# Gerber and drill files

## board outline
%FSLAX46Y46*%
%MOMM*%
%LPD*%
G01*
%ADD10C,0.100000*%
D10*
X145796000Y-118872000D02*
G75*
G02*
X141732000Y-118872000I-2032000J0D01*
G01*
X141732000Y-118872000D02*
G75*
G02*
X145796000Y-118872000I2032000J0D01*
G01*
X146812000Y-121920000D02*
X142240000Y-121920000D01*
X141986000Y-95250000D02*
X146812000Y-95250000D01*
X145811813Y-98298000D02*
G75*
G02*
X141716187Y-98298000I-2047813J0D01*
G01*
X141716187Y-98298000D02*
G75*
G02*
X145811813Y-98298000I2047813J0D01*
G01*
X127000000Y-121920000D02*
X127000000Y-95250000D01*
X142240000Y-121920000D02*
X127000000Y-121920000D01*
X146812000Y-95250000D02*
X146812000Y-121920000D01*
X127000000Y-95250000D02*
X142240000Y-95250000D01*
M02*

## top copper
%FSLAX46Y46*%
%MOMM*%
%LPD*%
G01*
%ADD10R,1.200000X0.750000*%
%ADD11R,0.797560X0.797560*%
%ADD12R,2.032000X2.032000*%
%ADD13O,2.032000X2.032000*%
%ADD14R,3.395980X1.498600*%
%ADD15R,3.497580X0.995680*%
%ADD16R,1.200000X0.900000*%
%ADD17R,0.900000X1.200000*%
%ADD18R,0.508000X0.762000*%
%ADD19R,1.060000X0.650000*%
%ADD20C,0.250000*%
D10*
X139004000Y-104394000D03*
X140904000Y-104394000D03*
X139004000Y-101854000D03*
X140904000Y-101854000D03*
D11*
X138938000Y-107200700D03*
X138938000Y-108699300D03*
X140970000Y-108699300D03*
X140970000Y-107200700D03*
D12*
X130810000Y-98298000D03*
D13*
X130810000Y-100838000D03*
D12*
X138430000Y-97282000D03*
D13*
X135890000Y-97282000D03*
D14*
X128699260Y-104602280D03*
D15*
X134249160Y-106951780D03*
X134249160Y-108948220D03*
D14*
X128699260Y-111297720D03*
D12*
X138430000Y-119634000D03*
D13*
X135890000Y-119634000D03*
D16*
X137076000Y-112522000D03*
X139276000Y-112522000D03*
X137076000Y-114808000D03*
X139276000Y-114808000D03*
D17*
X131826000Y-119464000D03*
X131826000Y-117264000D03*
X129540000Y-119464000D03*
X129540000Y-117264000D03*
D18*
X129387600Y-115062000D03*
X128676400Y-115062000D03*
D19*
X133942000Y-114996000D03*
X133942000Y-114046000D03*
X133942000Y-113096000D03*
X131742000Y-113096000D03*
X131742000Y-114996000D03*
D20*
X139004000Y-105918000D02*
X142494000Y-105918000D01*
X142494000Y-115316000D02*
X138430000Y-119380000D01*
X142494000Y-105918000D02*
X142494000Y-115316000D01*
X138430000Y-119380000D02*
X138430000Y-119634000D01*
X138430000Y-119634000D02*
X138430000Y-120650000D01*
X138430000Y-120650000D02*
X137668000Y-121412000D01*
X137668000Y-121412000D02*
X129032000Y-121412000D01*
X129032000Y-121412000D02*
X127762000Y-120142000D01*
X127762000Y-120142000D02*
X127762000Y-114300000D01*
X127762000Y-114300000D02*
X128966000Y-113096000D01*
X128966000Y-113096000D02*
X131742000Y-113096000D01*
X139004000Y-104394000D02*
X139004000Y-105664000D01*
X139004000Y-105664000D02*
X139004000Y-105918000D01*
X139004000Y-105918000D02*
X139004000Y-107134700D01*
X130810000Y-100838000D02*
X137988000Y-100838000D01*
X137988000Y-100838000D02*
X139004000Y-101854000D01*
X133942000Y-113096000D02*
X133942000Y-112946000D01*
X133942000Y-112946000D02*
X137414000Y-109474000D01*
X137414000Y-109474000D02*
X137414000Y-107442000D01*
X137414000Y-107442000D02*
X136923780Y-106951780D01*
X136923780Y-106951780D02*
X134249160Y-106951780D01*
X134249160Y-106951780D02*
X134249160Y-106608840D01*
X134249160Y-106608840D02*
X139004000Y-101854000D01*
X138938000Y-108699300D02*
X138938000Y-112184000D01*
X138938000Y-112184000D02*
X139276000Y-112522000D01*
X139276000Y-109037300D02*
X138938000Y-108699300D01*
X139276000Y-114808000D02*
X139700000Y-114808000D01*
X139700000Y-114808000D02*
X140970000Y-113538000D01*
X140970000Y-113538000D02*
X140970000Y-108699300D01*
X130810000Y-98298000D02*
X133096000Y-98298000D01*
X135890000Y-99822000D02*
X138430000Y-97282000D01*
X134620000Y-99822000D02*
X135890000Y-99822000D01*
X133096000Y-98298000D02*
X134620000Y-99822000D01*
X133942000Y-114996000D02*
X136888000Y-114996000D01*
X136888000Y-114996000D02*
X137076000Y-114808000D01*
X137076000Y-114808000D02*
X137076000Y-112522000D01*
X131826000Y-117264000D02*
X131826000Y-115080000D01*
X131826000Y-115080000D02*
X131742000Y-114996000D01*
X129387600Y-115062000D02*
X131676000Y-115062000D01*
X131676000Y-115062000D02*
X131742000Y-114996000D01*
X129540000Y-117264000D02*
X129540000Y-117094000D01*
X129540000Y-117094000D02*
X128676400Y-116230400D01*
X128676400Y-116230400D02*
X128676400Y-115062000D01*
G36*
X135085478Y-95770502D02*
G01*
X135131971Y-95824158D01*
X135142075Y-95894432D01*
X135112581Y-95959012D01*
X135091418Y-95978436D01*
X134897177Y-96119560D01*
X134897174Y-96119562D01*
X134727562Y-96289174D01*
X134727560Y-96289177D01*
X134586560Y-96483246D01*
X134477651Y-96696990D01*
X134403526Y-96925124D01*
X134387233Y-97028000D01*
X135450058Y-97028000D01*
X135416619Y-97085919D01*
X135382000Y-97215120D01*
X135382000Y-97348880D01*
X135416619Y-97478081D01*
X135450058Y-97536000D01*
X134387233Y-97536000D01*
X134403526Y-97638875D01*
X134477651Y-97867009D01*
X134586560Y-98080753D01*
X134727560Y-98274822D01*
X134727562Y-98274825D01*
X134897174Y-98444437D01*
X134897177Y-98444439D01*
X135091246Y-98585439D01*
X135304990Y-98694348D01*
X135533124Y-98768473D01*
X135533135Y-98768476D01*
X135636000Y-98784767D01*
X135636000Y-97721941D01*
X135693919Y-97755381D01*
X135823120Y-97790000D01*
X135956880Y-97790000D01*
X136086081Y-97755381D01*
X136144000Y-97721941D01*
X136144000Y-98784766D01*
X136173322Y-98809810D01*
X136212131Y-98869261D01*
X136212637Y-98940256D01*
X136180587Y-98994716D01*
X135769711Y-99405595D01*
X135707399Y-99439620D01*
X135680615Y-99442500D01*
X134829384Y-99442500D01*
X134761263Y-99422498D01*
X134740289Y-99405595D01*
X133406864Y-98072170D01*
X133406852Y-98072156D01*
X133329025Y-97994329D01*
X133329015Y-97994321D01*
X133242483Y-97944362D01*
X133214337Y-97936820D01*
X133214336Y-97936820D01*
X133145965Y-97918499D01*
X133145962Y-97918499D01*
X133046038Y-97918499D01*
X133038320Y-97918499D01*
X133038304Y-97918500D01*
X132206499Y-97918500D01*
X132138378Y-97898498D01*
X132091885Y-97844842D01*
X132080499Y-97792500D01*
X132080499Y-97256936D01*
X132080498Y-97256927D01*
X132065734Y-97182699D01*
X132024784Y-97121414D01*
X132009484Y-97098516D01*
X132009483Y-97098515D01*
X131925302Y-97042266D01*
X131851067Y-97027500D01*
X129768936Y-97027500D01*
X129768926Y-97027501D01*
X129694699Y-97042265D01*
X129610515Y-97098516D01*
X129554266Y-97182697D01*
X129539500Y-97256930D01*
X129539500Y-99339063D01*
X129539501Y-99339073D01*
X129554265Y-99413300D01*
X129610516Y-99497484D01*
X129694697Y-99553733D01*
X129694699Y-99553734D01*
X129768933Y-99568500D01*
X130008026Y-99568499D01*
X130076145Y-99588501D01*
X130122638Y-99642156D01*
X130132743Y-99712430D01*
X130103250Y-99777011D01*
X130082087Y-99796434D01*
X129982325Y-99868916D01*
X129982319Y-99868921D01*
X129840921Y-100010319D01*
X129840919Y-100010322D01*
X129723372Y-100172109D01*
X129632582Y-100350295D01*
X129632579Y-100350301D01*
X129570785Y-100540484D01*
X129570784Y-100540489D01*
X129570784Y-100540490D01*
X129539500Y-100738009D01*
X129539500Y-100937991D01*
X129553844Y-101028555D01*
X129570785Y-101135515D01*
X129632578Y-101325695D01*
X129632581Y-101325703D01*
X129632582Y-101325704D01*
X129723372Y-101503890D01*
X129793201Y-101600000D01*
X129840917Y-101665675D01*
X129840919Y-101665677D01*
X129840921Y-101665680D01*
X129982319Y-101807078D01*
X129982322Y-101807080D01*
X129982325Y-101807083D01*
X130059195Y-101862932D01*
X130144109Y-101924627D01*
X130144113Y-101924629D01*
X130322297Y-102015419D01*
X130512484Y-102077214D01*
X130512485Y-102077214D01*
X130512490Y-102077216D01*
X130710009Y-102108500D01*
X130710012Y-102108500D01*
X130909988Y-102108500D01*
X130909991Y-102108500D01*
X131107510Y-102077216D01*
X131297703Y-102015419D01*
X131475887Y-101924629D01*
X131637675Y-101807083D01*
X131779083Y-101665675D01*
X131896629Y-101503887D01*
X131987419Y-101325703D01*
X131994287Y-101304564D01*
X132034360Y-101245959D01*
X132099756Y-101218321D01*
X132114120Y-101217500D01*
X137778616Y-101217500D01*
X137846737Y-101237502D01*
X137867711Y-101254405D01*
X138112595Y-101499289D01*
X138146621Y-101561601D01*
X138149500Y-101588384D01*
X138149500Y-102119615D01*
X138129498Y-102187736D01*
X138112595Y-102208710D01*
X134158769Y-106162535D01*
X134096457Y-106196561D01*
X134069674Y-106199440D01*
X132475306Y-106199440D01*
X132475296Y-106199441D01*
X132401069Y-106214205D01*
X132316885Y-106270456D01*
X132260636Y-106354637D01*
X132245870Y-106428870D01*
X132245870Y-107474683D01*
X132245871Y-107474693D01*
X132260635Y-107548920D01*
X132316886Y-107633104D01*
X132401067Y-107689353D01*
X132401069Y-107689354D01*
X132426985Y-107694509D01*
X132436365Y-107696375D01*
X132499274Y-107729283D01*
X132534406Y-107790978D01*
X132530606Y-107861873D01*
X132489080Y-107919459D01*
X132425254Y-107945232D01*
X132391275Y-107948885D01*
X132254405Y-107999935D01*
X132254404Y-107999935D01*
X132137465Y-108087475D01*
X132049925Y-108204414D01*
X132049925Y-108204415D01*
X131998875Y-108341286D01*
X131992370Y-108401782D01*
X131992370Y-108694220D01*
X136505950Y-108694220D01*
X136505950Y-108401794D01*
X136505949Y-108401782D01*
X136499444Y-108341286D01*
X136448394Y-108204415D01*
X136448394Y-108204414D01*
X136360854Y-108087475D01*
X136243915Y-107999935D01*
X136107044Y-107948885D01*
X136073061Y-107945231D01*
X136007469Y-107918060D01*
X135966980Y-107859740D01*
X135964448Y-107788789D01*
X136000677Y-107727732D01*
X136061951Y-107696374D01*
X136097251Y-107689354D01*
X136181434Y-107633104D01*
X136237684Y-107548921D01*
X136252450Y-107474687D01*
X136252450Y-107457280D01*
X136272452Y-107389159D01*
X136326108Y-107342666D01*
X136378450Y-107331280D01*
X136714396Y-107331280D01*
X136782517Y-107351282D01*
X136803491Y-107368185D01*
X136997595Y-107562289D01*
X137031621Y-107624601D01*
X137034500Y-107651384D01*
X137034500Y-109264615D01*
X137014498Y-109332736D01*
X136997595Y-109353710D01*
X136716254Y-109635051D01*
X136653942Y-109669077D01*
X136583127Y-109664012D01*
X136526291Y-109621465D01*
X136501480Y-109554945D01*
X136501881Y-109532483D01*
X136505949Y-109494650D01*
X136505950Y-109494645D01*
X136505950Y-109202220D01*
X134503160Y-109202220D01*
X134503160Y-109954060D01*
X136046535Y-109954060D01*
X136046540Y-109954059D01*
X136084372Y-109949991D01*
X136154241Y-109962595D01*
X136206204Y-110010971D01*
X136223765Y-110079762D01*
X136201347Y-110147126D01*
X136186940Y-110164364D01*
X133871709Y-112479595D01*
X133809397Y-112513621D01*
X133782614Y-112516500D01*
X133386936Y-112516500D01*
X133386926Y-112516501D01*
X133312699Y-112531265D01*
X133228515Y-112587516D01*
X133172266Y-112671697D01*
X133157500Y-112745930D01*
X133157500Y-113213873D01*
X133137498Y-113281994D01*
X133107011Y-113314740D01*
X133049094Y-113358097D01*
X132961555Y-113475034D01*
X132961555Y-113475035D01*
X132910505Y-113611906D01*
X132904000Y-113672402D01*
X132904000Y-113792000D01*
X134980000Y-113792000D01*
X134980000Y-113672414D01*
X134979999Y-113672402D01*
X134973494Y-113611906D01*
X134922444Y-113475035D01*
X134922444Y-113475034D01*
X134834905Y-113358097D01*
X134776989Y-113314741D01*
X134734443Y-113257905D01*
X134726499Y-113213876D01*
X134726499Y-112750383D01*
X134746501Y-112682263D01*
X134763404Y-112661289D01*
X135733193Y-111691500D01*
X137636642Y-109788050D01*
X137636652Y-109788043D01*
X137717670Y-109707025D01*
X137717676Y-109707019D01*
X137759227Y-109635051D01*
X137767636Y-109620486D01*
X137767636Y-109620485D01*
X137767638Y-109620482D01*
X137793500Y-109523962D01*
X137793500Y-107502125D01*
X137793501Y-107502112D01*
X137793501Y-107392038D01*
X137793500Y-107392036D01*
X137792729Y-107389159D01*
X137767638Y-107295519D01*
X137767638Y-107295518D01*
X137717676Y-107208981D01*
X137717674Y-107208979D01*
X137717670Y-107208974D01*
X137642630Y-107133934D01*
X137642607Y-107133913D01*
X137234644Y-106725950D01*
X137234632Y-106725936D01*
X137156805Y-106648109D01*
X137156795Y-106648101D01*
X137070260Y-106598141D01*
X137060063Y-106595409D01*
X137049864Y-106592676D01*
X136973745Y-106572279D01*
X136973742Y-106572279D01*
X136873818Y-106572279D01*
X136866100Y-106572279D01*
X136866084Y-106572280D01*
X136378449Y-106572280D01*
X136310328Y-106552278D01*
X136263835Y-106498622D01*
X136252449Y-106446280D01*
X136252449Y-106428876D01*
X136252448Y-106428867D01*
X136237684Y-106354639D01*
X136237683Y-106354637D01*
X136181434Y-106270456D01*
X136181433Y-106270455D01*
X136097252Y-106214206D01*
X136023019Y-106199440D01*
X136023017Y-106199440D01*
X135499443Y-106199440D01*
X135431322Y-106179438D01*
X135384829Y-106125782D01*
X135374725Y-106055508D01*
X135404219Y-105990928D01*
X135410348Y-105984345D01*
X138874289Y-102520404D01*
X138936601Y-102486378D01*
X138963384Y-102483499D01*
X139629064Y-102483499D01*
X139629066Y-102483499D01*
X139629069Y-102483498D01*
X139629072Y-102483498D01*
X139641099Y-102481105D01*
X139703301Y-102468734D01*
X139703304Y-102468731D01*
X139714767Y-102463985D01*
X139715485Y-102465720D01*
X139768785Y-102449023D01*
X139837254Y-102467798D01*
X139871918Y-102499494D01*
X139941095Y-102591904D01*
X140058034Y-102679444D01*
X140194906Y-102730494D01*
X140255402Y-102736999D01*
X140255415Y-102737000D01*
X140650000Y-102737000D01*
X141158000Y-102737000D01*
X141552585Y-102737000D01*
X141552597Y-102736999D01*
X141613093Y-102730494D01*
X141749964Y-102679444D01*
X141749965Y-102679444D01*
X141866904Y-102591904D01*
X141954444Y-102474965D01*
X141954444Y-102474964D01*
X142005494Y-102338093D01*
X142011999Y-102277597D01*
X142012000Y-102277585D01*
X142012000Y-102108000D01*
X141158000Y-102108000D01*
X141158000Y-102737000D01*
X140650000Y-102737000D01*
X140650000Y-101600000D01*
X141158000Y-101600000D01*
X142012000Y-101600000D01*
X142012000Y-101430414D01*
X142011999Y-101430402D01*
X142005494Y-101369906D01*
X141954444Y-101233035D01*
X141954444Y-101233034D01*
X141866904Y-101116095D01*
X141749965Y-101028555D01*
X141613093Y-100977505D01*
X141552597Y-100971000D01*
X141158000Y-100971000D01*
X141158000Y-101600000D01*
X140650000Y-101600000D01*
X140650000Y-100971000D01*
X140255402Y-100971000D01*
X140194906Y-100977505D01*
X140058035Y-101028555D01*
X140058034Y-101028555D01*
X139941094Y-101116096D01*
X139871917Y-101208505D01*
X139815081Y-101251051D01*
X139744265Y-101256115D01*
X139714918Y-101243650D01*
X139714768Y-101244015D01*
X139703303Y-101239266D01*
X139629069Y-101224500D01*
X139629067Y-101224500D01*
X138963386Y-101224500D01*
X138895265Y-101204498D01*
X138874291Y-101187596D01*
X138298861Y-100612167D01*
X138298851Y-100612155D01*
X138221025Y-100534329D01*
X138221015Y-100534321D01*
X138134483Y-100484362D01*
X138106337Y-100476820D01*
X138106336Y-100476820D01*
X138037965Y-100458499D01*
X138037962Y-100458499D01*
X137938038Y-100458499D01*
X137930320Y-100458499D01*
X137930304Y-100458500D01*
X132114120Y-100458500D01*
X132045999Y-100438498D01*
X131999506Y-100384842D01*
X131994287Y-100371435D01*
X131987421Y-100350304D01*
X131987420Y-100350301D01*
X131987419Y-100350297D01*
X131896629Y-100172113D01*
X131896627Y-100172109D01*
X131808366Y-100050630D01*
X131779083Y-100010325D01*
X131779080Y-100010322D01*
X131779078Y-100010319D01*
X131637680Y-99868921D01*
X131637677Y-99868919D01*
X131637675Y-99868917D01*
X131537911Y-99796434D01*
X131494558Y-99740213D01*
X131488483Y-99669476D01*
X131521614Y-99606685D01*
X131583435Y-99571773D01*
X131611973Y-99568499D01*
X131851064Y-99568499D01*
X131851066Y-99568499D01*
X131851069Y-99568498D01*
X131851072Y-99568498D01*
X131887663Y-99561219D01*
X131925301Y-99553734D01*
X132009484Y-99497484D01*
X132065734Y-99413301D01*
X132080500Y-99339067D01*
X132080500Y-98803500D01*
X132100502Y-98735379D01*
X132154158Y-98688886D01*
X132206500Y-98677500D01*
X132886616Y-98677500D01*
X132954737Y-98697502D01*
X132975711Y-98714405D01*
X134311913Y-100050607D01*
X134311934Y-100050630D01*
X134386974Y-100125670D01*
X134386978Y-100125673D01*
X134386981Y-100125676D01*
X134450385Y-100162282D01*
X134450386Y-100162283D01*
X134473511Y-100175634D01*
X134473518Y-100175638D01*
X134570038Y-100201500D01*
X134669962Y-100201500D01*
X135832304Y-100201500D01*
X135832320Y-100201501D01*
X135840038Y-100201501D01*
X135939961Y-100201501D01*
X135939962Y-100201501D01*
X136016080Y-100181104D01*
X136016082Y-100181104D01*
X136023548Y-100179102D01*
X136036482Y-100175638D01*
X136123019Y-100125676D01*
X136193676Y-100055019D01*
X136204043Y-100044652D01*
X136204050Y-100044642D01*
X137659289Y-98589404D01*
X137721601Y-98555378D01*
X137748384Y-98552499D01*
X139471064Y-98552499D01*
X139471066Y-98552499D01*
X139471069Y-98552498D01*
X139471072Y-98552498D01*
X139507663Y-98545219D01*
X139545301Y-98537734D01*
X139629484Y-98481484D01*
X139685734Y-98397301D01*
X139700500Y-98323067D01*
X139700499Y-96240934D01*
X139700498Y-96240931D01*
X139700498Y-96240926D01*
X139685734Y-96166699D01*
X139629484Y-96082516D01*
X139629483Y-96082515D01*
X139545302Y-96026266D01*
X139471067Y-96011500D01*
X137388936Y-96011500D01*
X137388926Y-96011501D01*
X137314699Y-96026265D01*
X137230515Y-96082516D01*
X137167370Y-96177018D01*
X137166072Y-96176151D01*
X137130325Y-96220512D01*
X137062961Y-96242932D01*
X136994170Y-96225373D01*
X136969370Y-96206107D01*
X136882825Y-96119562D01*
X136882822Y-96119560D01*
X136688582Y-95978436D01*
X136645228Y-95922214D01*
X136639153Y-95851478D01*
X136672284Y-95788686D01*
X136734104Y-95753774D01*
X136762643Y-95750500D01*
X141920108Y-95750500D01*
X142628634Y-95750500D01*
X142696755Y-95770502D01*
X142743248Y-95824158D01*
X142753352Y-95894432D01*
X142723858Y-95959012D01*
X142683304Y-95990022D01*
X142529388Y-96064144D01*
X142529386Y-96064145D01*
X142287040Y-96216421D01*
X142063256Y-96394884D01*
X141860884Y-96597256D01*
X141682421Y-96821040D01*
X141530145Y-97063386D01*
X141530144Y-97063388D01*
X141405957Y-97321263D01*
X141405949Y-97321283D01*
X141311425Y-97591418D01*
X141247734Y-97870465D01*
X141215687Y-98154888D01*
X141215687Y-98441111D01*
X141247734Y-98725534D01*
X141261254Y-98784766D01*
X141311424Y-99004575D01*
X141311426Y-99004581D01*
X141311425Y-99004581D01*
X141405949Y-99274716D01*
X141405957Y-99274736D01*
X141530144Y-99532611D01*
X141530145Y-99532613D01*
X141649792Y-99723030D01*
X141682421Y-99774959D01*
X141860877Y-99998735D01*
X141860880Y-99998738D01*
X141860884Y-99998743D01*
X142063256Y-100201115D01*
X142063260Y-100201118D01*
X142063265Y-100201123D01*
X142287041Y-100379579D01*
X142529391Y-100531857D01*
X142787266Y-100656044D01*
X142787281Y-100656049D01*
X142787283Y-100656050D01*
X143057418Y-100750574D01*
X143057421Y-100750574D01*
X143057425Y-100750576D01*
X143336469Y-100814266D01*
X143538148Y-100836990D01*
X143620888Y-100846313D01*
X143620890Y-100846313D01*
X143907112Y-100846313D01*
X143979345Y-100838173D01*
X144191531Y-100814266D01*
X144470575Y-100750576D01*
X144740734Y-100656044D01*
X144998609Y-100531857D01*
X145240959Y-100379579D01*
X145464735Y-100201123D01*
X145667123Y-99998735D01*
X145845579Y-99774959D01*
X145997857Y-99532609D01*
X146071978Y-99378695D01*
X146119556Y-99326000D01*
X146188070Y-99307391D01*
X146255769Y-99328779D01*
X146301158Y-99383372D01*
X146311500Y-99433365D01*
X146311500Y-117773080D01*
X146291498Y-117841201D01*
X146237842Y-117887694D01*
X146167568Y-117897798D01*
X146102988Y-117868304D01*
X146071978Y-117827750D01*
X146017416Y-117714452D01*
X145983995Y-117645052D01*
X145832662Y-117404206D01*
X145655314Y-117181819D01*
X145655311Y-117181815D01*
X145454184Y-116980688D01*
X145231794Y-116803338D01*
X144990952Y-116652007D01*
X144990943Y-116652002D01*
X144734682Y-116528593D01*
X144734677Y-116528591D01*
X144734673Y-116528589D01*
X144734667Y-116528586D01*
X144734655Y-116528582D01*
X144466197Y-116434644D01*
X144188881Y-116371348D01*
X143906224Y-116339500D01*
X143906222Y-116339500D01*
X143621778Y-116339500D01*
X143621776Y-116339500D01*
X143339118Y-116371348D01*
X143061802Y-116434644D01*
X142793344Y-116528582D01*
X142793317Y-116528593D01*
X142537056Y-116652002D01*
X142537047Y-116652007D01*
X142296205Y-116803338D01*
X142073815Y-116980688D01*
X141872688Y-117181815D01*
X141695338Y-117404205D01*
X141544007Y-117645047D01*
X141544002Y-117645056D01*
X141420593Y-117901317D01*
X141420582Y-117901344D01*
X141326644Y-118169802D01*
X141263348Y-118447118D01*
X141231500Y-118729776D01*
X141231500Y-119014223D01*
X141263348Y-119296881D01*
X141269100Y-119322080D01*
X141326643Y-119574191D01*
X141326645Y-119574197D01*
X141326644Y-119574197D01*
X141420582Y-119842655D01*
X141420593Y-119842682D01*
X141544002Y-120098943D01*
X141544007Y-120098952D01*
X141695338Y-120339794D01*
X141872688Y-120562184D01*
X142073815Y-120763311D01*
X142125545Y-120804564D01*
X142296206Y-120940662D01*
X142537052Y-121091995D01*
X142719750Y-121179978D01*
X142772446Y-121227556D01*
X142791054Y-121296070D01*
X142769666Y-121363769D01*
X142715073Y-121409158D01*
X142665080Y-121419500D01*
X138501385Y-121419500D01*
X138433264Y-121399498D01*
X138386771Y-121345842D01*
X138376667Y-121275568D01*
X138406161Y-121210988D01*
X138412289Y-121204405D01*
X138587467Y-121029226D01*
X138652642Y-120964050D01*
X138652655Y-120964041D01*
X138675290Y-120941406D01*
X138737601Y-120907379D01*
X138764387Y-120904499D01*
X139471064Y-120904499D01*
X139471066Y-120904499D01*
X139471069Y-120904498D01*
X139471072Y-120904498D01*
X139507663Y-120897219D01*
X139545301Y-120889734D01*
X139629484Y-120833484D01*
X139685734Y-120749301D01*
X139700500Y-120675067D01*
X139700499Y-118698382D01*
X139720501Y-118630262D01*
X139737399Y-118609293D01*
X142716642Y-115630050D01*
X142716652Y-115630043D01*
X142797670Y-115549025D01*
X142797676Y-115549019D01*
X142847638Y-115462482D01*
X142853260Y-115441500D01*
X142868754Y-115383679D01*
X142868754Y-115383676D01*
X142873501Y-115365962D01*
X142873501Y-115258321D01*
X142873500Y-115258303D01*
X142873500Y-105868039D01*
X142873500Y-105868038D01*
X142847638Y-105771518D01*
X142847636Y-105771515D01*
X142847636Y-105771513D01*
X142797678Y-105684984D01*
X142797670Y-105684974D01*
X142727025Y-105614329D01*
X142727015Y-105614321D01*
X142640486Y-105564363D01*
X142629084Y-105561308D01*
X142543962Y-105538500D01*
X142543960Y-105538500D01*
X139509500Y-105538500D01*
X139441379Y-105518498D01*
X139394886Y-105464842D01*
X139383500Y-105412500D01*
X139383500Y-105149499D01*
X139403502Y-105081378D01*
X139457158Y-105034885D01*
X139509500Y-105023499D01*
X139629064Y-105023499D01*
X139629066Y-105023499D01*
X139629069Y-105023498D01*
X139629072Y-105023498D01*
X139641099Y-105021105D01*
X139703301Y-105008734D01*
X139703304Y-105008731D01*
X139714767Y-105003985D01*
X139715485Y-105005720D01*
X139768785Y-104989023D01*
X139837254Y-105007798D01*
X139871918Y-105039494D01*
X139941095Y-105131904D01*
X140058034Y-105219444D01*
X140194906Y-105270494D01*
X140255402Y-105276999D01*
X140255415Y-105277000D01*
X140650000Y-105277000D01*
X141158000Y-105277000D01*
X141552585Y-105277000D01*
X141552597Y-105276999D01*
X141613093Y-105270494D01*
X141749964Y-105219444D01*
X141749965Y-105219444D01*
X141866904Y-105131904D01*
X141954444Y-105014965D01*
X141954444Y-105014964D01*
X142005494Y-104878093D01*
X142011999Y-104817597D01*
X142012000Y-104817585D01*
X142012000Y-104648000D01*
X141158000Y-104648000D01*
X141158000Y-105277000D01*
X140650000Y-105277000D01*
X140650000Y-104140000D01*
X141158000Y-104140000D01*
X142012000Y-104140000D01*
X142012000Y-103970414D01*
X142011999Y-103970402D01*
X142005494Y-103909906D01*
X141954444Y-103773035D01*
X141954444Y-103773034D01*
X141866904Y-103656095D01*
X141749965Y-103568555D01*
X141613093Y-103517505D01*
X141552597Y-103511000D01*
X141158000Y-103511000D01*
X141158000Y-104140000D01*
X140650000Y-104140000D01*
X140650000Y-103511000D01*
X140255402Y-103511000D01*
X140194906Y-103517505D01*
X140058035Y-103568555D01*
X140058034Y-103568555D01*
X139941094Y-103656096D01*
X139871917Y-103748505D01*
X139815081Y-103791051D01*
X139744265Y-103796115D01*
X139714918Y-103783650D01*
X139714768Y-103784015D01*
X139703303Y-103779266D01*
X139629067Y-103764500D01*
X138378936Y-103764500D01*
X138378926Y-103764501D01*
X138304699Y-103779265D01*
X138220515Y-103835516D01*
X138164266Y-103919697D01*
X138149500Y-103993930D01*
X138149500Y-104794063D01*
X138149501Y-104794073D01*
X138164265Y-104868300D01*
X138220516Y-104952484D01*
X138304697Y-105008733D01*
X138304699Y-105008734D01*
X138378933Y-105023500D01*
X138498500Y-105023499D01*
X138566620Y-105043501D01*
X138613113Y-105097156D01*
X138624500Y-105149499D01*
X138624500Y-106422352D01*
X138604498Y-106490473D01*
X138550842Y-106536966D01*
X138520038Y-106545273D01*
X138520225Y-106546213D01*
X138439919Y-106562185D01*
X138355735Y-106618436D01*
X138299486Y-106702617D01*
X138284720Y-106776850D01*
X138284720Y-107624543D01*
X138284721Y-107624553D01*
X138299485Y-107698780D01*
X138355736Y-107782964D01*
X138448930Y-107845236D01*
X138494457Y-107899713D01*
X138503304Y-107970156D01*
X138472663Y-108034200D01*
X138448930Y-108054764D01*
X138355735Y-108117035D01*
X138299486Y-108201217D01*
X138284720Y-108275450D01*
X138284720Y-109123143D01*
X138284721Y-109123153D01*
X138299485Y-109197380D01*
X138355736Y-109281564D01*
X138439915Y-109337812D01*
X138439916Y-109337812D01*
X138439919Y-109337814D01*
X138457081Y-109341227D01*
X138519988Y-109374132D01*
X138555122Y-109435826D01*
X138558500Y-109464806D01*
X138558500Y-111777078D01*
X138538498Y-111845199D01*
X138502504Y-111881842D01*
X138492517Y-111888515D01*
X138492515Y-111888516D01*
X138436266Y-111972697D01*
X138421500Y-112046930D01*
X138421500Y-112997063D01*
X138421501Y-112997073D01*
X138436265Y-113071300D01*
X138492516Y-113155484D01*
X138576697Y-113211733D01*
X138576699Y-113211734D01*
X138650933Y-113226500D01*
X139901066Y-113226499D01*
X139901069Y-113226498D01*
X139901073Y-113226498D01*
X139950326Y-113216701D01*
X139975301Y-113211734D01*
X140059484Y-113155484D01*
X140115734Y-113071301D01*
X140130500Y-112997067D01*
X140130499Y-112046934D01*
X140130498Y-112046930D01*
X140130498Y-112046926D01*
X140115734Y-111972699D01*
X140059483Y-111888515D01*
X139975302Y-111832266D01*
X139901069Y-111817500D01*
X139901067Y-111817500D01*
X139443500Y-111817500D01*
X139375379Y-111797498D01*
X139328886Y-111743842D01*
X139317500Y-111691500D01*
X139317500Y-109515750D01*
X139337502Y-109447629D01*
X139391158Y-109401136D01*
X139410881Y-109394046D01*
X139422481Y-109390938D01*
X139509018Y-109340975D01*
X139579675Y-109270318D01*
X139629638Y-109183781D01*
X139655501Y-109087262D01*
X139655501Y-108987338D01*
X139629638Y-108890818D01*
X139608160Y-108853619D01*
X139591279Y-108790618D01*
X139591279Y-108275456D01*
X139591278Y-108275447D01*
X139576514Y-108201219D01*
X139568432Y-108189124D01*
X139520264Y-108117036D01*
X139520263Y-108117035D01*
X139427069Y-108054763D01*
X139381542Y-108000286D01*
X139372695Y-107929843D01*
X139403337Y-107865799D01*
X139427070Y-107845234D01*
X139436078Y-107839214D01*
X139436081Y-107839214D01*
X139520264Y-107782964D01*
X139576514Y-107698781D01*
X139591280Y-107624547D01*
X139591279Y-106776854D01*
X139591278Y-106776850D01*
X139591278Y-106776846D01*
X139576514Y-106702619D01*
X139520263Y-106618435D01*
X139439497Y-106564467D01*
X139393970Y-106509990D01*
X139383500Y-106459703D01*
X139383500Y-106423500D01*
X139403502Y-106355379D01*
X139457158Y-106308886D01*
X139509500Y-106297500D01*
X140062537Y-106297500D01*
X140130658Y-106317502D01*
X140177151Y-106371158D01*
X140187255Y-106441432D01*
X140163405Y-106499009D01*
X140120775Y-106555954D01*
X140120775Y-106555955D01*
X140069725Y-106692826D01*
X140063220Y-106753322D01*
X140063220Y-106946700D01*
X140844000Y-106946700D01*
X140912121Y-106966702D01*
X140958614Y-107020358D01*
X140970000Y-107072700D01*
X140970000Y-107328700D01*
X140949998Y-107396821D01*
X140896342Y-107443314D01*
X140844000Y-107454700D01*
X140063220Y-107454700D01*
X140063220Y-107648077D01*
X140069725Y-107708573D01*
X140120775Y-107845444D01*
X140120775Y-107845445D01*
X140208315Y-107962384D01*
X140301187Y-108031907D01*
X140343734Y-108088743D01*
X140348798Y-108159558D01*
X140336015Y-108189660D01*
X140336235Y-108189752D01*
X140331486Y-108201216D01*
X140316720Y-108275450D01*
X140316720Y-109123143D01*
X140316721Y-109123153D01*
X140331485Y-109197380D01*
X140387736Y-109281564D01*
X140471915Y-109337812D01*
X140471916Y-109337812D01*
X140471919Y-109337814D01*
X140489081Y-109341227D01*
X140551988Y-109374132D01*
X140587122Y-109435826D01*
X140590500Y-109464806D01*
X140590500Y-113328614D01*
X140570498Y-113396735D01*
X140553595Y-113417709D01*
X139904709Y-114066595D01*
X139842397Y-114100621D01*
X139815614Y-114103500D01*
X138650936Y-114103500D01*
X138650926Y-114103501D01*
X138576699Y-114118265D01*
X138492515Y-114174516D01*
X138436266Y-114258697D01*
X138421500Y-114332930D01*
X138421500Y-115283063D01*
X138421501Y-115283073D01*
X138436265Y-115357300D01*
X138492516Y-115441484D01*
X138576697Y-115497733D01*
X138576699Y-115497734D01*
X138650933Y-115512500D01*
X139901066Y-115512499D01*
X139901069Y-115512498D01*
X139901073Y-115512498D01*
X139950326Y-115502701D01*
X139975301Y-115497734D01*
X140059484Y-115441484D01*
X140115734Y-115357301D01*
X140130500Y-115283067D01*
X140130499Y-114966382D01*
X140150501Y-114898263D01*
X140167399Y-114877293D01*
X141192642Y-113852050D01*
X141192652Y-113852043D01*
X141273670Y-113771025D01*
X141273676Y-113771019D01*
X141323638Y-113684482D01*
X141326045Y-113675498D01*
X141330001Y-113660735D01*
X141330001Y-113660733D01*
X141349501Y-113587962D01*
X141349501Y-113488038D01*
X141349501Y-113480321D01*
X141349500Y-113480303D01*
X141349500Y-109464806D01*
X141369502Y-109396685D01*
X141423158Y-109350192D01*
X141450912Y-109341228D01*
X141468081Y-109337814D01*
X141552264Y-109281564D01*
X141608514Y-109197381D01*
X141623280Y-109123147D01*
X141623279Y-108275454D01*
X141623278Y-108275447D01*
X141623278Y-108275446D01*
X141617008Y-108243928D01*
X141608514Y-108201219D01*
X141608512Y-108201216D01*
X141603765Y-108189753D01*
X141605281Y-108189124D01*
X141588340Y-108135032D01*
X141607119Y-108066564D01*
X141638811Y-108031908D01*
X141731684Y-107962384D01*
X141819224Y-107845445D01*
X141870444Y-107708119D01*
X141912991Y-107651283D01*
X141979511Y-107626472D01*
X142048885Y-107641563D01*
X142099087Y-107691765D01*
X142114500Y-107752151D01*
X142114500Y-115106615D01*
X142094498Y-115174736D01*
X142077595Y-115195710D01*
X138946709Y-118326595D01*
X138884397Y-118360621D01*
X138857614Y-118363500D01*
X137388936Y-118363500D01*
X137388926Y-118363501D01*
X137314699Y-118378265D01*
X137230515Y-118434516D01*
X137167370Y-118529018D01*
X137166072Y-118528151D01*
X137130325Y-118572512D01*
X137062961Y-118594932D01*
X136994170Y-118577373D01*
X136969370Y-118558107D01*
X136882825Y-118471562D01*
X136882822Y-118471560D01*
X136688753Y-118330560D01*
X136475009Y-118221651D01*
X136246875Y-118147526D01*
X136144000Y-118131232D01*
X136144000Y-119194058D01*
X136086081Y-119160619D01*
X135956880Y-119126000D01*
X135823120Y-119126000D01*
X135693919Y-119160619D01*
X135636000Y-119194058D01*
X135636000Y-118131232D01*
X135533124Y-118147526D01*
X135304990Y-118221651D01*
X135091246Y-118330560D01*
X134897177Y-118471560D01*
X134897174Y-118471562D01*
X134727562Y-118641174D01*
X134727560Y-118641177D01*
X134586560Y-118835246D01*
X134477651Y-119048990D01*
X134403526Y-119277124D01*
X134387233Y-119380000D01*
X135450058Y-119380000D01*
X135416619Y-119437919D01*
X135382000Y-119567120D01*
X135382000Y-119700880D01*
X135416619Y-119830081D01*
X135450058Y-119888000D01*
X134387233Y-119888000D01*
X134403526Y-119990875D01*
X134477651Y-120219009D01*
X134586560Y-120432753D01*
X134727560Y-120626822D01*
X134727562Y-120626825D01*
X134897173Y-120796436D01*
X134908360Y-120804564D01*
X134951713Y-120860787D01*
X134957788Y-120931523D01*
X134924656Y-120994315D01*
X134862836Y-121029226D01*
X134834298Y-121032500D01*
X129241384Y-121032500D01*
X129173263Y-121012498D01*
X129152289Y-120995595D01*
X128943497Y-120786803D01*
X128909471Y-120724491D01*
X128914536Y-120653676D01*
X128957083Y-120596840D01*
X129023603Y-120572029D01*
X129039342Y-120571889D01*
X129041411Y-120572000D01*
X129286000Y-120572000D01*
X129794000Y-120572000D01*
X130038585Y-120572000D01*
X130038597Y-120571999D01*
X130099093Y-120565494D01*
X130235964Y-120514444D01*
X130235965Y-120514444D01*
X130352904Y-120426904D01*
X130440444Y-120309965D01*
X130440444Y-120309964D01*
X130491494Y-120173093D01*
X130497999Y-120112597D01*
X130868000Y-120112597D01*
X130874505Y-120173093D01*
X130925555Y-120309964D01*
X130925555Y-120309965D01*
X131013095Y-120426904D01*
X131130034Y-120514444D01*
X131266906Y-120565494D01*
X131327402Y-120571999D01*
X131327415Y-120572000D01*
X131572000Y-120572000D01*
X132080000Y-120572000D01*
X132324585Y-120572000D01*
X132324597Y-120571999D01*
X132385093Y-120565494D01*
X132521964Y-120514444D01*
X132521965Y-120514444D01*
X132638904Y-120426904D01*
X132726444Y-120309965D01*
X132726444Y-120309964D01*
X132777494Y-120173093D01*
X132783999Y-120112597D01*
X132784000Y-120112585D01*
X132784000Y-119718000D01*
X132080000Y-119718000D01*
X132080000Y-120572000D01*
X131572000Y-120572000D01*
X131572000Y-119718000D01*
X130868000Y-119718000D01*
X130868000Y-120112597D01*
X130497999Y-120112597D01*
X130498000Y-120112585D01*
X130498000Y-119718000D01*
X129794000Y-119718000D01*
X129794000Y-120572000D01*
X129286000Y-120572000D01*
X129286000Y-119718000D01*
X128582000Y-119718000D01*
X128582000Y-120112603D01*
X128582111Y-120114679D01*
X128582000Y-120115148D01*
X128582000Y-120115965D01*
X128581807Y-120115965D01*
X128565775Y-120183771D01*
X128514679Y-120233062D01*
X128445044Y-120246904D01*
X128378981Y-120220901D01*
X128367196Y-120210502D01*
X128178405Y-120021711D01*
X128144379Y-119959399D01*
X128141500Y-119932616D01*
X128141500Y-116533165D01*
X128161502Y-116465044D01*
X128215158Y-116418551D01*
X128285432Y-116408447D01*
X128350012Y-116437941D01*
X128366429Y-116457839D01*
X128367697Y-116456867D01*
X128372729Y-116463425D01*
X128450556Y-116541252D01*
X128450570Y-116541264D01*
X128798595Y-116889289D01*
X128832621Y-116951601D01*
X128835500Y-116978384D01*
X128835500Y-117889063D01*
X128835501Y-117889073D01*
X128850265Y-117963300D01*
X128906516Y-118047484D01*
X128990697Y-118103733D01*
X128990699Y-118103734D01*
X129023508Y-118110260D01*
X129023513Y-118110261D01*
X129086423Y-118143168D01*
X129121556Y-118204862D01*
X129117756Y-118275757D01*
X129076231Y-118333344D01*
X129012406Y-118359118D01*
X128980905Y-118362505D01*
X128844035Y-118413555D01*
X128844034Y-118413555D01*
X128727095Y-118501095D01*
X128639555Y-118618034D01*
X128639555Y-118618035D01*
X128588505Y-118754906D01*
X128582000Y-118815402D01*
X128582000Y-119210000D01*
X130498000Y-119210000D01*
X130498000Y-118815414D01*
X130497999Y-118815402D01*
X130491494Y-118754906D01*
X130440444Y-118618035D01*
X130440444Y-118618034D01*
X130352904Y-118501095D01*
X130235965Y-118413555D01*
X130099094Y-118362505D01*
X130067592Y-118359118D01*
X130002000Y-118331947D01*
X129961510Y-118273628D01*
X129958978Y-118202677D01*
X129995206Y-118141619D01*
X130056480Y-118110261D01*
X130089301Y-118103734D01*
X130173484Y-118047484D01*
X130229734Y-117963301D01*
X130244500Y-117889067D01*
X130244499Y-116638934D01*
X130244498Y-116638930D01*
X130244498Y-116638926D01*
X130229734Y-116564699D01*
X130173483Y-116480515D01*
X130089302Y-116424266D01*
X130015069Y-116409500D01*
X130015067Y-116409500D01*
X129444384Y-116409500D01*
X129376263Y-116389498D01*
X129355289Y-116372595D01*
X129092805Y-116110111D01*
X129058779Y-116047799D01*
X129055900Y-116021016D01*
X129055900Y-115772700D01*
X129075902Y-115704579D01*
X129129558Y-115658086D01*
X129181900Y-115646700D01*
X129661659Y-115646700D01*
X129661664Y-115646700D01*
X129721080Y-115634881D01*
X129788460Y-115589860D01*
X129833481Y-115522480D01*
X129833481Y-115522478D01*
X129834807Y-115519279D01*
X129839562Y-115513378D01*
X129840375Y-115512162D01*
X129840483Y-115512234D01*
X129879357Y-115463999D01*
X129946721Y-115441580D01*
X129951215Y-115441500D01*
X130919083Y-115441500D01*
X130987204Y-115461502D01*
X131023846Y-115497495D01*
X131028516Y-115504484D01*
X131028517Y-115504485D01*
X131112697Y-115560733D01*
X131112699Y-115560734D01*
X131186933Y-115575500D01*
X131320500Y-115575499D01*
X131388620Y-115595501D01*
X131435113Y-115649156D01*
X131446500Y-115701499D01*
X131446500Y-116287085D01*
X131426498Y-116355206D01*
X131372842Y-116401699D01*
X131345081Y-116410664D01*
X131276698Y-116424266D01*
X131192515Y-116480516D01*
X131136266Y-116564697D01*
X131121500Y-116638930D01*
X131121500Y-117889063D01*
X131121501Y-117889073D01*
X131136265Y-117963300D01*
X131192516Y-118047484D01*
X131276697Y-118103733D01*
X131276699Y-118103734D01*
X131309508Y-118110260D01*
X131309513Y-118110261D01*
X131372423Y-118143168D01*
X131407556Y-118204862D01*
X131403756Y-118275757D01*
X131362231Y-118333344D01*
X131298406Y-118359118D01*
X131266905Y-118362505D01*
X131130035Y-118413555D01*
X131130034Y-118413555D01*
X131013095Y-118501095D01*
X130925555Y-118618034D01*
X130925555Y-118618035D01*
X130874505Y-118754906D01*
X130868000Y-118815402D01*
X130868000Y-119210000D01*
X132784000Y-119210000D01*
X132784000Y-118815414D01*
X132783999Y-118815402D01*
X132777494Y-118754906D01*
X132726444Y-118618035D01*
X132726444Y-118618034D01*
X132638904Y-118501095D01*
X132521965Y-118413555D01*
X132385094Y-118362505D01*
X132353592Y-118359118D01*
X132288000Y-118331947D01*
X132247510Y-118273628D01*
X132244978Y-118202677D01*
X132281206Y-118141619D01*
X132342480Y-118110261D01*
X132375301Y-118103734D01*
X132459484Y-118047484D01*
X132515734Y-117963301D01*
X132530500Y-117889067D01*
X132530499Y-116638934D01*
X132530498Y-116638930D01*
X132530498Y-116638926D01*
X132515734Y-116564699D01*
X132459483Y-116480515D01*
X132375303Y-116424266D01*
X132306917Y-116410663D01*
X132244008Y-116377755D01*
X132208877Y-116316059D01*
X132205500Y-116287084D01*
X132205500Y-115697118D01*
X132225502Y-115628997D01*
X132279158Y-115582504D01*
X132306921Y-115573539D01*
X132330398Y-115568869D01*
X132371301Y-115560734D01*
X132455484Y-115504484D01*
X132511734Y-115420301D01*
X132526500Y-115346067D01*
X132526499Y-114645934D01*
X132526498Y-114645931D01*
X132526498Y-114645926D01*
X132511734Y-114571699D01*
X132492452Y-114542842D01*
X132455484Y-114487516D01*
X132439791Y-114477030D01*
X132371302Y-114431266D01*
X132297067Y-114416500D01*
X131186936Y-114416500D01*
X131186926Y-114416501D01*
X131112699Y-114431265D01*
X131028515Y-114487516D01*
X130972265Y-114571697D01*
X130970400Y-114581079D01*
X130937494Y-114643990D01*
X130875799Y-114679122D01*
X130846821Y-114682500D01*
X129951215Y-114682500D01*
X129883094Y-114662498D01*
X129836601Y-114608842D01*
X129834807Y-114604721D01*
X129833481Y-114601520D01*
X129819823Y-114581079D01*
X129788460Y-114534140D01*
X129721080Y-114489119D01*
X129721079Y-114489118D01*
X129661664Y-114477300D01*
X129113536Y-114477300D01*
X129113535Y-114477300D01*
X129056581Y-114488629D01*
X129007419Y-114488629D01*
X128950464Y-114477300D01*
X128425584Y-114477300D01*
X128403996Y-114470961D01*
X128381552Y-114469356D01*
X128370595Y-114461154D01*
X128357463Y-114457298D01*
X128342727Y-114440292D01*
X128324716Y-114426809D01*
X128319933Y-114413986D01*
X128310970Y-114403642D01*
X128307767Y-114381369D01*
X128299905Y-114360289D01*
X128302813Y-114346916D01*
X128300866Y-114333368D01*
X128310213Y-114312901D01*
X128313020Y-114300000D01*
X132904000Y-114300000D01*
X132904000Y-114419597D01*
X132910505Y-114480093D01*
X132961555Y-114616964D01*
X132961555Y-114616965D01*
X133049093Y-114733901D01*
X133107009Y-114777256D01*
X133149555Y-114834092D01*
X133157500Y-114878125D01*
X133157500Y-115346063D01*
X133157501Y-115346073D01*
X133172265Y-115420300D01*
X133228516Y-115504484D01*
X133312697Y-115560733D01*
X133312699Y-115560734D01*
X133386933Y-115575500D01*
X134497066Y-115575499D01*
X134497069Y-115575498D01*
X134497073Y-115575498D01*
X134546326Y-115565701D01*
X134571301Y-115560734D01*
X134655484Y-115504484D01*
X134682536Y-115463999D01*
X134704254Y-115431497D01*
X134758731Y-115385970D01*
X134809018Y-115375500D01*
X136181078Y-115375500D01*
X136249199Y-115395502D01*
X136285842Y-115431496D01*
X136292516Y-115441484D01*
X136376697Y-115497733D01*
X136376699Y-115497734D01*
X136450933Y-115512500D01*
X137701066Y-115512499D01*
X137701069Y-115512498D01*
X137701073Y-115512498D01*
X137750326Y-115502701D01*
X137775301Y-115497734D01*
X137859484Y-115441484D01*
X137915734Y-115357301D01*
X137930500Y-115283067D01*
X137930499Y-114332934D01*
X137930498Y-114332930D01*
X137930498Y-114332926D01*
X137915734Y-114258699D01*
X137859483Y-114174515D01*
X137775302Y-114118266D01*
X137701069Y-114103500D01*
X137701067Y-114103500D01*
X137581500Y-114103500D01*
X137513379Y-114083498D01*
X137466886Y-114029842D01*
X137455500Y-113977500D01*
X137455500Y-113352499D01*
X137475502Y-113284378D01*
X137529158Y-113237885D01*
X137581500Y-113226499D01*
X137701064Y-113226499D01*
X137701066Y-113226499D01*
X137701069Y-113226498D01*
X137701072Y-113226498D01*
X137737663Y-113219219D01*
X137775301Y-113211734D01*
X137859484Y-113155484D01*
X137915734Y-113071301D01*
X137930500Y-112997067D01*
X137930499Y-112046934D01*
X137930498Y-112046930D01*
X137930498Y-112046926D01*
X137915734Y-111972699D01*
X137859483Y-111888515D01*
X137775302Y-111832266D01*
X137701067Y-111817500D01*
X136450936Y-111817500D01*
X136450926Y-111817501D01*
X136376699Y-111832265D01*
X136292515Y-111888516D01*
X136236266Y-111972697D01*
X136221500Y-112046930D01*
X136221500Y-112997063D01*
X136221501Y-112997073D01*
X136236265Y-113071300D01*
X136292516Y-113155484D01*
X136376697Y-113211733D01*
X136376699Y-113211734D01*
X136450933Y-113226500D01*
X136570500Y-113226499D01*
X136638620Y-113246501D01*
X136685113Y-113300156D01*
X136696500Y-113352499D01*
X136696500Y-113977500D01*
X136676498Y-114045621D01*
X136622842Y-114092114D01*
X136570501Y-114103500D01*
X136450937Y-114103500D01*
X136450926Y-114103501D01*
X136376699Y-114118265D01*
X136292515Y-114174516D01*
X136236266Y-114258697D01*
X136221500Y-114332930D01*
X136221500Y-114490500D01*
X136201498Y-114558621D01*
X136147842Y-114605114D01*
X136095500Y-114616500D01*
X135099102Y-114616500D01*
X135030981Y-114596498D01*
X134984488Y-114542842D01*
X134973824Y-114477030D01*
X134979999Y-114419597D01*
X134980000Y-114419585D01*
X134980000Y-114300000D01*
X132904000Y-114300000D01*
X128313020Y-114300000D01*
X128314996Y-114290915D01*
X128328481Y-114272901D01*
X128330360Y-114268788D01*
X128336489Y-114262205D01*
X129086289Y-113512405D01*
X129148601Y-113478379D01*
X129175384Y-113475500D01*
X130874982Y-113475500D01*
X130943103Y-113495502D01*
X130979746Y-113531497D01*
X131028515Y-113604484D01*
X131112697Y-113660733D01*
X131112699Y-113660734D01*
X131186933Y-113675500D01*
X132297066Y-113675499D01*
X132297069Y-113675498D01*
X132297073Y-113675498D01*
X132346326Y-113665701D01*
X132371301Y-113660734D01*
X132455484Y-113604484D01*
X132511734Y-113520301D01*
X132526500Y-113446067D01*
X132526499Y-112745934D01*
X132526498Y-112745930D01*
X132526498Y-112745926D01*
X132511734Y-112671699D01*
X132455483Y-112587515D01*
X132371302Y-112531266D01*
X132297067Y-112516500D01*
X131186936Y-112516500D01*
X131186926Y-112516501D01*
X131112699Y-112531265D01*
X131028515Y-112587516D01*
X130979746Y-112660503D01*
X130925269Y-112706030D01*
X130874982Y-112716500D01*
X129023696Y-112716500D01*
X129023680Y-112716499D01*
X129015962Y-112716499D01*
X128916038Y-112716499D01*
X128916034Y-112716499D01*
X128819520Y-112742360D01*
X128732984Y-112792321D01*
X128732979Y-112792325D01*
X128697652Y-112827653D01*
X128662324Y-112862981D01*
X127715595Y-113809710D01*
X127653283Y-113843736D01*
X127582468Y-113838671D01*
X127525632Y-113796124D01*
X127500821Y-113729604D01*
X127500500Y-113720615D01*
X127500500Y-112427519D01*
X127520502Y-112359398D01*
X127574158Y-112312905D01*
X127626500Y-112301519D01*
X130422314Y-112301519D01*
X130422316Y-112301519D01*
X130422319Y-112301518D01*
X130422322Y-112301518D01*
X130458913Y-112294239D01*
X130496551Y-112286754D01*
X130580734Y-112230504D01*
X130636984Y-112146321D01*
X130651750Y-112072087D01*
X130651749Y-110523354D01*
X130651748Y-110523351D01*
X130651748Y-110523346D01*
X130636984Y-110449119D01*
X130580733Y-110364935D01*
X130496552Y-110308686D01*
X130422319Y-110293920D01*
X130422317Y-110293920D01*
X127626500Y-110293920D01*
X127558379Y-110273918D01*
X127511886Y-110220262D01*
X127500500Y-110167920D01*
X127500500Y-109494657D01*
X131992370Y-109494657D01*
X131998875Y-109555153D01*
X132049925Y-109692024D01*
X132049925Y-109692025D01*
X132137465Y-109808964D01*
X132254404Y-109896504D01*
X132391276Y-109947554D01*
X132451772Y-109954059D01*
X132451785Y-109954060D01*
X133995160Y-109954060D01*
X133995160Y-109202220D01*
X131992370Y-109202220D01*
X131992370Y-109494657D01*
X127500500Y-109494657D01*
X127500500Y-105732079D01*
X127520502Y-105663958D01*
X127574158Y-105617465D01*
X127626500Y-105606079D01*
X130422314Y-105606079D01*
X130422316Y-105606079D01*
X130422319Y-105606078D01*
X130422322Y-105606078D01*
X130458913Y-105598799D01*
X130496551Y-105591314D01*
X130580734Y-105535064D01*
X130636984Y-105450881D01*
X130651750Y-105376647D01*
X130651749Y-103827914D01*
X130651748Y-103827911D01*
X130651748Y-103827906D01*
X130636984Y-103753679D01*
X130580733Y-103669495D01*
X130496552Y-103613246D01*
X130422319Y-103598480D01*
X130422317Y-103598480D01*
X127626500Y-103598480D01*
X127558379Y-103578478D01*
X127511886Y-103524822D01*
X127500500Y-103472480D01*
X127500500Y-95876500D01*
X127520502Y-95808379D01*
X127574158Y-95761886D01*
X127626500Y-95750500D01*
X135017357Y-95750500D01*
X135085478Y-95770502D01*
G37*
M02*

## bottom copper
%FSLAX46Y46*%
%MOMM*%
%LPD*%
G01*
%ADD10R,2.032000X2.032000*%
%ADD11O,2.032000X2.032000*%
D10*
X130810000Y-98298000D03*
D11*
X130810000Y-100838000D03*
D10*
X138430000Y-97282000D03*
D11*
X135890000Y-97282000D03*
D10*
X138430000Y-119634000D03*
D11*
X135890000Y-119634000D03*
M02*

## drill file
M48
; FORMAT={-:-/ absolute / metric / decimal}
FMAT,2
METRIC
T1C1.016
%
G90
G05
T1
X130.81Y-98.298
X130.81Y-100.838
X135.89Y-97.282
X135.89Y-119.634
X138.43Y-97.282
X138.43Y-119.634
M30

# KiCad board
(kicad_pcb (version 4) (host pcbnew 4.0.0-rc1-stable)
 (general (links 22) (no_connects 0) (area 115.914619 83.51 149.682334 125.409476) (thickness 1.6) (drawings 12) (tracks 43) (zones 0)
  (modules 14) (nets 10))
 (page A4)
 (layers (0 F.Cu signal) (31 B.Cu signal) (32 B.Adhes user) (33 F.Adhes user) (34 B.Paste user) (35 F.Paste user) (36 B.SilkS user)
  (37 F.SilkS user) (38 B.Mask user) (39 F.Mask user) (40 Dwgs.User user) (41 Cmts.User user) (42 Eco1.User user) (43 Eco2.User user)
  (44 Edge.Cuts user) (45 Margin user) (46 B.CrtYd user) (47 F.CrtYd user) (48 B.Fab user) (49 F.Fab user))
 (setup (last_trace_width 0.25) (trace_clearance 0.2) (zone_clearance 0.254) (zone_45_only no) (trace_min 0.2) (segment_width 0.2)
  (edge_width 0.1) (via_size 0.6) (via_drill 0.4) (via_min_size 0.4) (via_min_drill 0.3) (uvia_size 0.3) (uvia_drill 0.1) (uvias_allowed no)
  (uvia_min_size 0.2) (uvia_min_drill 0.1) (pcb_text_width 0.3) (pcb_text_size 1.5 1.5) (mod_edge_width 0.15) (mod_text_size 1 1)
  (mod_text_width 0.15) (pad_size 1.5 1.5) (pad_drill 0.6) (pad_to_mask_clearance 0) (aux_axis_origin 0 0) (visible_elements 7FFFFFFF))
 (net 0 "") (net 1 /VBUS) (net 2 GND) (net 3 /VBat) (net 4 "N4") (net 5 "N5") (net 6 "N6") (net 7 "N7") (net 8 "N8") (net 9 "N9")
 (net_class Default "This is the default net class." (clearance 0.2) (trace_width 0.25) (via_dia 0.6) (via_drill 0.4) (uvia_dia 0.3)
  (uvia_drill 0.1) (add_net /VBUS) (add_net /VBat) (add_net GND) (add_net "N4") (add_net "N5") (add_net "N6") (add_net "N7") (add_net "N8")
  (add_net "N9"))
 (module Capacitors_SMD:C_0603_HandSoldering (layer F.Cu) (at 139.954 104.394)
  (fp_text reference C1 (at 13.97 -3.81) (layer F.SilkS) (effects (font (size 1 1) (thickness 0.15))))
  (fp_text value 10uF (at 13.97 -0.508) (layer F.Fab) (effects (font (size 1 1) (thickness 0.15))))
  (pad 1 smd rect (at -0.95 0) (size 1.2 0.75) (layers F.Cu F.Paste F.Mask) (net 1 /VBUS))
  (pad 2 smd rect (at 0.95 0) (size 1.2 0.75) (layers F.Cu F.Paste F.Mask) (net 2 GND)))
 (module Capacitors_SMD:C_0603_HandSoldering (layer F.Cu) (at 139.954 101.854)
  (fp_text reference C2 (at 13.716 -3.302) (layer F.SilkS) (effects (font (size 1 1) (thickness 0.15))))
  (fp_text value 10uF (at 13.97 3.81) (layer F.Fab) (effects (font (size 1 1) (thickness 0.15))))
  (pad 1 smd rect (at -0.95 0) (size 1.2 0.75) (layers F.Cu F.Paste F.Mask) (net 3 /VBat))
  (pad 2 smd rect (at 0.95 0) (size 1.2 0.75) (layers F.Cu F.Paste F.Mask) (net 2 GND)))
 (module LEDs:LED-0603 (layer F.Cu) (at 138.938 107.95 90)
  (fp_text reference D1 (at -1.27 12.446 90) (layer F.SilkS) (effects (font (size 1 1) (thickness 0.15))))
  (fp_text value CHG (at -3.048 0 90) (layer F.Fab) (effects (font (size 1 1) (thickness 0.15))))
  (pad 2 smd rect (at 0.7493 0 270) (size 0.79756 0.79756) (layers F.Cu F.Paste F.Mask) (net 1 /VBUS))
  (pad 1 smd rect (at -0.7493 0 270) (size 0.79756 0.79756) (layers F.Cu F.Paste F.Mask) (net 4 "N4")))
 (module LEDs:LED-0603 (layer F.Cu) (at 140.97 107.95 270)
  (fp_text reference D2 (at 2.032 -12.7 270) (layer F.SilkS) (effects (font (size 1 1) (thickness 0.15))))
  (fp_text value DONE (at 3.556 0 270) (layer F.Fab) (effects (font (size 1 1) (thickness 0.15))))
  (pad 2 smd rect (at 0.7493 0 90) (size 0.79756 0.79756) (layers F.Cu F.Paste F.Mask) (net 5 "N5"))
  (pad 1 smd rect (at -0.7493 0 90) (size 0.79756 0.79756) (layers F.Cu F.Paste F.Mask) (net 2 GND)))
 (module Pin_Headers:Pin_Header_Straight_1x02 (layer F.Cu) (at 130.81 98.298)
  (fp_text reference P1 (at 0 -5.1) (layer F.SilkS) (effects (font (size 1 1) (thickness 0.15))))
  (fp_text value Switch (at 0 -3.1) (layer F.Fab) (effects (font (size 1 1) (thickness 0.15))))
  (pad 1 thru_hole rect (at 0 0) (size 2.032 2.032) (drill 1.016) (layers *.Cu *.Mask F.SilkS) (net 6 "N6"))
  (pad 2 thru_hole oval (at 0 2.54) (size 2.032 2.032) (drill 1.016) (layers *.Cu *.Mask F.SilkS) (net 3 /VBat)))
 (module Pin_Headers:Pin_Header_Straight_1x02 (layer F.Cu) (at 138.43 97.282 270)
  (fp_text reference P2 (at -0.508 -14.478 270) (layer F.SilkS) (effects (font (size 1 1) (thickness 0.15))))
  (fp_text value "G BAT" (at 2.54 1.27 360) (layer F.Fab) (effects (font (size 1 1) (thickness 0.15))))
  (pad 1 thru_hole rect (at 0 0 270) (size 2.032 2.032) (drill 1.016) (layers *.Cu *.Mask F.SilkS) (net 6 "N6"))
  (pad 2 thru_hole oval (at 0 2.54 270) (size 2.032 2.032) (drill 1.016) (layers *.Cu *.Mask F.SilkS) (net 2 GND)))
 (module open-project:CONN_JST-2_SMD (layer F.Cu) (at 127 107.95 270)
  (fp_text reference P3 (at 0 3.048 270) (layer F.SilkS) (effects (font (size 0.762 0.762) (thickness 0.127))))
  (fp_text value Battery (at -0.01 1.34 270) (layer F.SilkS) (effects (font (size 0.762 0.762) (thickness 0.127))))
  (pad "" smd rect (at -3.34772 -1.69926 270) (size 1.4986 3.39598) (layers F.Cu F.Paste F.Mask))
  (pad 1 smd rect (at -0.99822 -7.24916 270) (size 0.99568 3.49758) (layers F.Cu F.Paste F.Mask) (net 3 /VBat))
  (pad 2 smd rect (at 0.99822 -7.24916 270) (size 0.99568 3.49758) (layers F.Cu F.Paste F.Mask) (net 2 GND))
  (pad "" smd rect (at 3.34772 -1.69926 270) (size 1.4986 3.39598) (layers F.Cu F.Paste F.Mask)))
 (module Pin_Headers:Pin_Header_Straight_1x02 (layer F.Cu) (at 138.43 119.634 270)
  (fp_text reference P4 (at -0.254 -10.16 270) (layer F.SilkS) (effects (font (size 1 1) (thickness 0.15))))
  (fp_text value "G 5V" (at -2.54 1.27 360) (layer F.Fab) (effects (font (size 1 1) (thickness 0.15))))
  (pad 1 thru_hole rect (at 0 0 270) (size 2.032 2.032) (drill 1.016) (layers *.Cu *.Mask F.SilkS) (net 1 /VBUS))
  (pad 2 thru_hole oval (at 0 2.54 270) (size 2.032 2.032) (drill 1.016) (layers *.Cu *.Mask F.SilkS) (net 2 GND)))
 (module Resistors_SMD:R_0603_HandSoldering (layer F.Cu) (at 138.176 112.522)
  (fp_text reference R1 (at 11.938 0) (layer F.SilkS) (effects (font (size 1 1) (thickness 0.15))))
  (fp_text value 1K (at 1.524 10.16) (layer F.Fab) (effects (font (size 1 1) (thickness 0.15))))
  (pad 1 smd rect (at -1.1 0) (size 1.2 0.9) (layers F.Cu F.Paste F.Mask) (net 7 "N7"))
  (pad 2 smd rect (at 1.1 0) (size 1.2 0.9) (layers F.Cu F.Paste F.Mask) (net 4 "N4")))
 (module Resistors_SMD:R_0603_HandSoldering (layer F.Cu) (at 138.176 114.808)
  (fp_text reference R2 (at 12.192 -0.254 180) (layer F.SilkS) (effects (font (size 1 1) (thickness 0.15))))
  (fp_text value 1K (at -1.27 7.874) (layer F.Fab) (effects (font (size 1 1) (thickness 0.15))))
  (pad 1 smd rect (at -1.1 0) (size 1.2 0.9) (layers F.Cu F.Paste F.Mask) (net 7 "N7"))
  (pad 2 smd rect (at 1.1 0) (size 1.2 0.9) (layers F.Cu F.Paste F.Mask) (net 5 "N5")))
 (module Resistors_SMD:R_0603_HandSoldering (layer F.Cu) (at 131.826 118.364 90)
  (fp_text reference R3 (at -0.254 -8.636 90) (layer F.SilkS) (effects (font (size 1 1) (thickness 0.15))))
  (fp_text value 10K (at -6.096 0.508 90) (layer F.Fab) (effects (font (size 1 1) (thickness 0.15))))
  (pad 1 smd rect (at -1.1 0 90) (size 1.2 0.9) (layers F.Cu F.Paste F.Mask) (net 2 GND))
  (pad 2 smd rect (at 1.1 0 90) (size 1.2 0.9) (layers F.Cu F.Paste F.Mask) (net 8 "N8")))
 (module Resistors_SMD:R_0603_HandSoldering (layer F.Cu) (at 129.54 118.364 90)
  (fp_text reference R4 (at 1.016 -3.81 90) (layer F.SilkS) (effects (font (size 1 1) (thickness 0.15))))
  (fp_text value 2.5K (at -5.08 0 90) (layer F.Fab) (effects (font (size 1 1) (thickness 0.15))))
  (pad 1 smd rect (at -1.1 0 90) (size 1.2 0.9) (layers F.Cu F.Paste F.Mask) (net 2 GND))
  (pad 2 smd rect (at 1.1 0 90) (size 1.2 0.9) (layers F.Cu F.Paste F.Mask) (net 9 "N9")))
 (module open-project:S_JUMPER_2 (layer F.Cu) (at 129.032 115.062 180)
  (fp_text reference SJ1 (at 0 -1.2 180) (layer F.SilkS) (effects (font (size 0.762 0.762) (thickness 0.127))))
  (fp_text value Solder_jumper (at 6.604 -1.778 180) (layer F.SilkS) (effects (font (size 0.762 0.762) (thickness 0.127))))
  (pad 1 smd rect (at -0.3556 0 180) (size 0.508 0.762) (layers F.Cu F.Paste F.Mask) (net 8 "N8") (clearance 0.2032))
  (pad 2 smd rect (at 0.3556 0 180) (size 0.508 0.762) (layers F.Cu F.Paste F.Mask) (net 9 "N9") (clearance 0.2032)))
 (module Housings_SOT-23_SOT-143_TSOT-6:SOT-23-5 (layer F.Cu) (at 132.842 114.046 180)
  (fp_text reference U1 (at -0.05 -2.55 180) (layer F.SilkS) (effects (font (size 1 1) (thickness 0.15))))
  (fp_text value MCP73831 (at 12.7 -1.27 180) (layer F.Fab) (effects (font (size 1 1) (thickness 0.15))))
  (pad 1 smd rect (at -1.1 -0.95 180) (size 1.06 0.65) (layers F.Cu F.Paste F.Mask) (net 7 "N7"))
  (pad 2 smd rect (at -1.1 0 180) (size 1.06 0.65) (layers F.Cu F.Paste F.Mask) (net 2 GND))
  (pad 3 smd rect (at -1.1 0.95 180) (size 1.06 0.65) (layers F.Cu F.Paste F.Mask) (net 3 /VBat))
  (pad 4 smd rect (at 1.1 0.95 180) (size 1.06 0.65) (layers F.Cu F.Paste F.Mask) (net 1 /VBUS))
  (pad 5 smd rect (at 1.1 -0.95 180) (size 1.06 0.65) (layers F.Cu F.Paste F.Mask) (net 8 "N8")))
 (gr_circle (center 143.764 118.872) (end 145.796 118.872) (layer Edge.Cuts) (width 0.1))
 (gr_line (start 146.812 121.92) (end 142.24 121.92) (angle 90) (layer Edge.Cuts) (width 0.1))
 (gr_line (start 141.986 95.25) (end 146.812 95.25) (angle 90) (layer Edge.Cuts) (width 0.1))
 (gr_circle (center 143.764 98.298) (end 145.796 98.044) (layer Edge.Cuts) (width 0.1))
 (gr_line (start 127 121.92) (end 127 95.25) (angle 90) (layer Edge.Cuts) (width 0.1))
 (gr_line (start 142.24 121.92) (end 127 121.92) (angle 90) (layer Edge.Cuts) (width 0.1))
 (gr_line (start 146.812 95.25) (end 146.812 121.92) (angle 90) (layer Edge.Cuts) (width 0.1))
 (gr_line (start 127 95.25) (end 142.24 95.25) (angle 90) (layer Edge.Cuts) (width 0.1))
 (segment (start 139.004 105.918) (end 142.494 105.918) (width 0.25) (layer F.Cu) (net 1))
 (segment (start 142.494 115.316) (end 138.43 119.38) (width 0.25) (layer F.Cu) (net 1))
 (segment (start 142.494 105.918) (end 142.494 115.316) (width 0.25) (layer F.Cu) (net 1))
 (segment (start 138.43 119.38) (end 138.43 119.634) (width 0.25) (layer F.Cu) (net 1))
 (segment (start 138.43 119.634) (end 138.43 120.65) (width 0.25) (layer F.Cu) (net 1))
 (segment (start 138.43 120.65) (end 137.668 121.412) (width 0.25) (layer F.Cu) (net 1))
 (segment (start 137.668 121.412) (end 129.032 121.412) (width 0.25) (layer F.Cu) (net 1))
 (segment (start 129.032 121.412) (end 127.762 120.142) (width 0.25) (layer F.Cu) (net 1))
 (segment (start 127.762 120.142) (end 127.762 114.3) (width 0.25) (layer F.Cu) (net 1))
 (segment (start 127.762 114.3) (end 128.966 113.096) (width 0.25) (layer F.Cu) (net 1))
 (segment (start 128.966 113.096) (end 131.742 113.096) (width 0.25) (layer F.Cu) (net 1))
 (segment (start 139.004 104.394) (end 139.004 105.664) (width 0.25) (layer F.Cu) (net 1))
 (segment (start 139.004 105.664) (end 139.004 105.918) (width 0.25) (layer F.Cu) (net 1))
 (segment (start 139.004 105.918) (end 139.004 107.1347) (width 0.25) (layer F.Cu) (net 1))
 (segment (start 130.81 100.838) (end 137.988 100.838) (width 0.25) (layer F.Cu) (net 3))
 (segment (start 137.988 100.838) (end 139.004 101.854) (width 0.25) (layer F.Cu) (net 3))
 (segment (start 133.942 113.096) (end 133.942 112.946) (width 0.25) (layer F.Cu) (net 3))
 (segment (start 133.942 112.946) (end 137.414 109.474) (width 0.25) (layer F.Cu) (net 3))
 (segment (start 137.414 109.474) (end 137.414 107.442) (width 0.25) (layer F.Cu) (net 3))
 (segment (start 137.414 107.442) (end 136.92378 106.95178) (width 0.25) (layer F.Cu) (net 3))
 (segment (start 136.92378 106.95178) (end 134.24916 106.95178) (width 0.25) (layer F.Cu) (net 3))
 (segment (start 134.24916 106.95178) (end 134.24916 106.60884) (width 0.25) (layer F.Cu) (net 3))
 (segment (start 134.24916 106.60884) (end 139.004 101.854) (width 0.25) (layer F.Cu) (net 3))
 (segment (start 138.938 108.6993) (end 138.938 112.184) (width 0.25) (layer F.Cu) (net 4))
 (segment (start 138.938 112.184) (end 139.276 112.522) (width 0.25) (layer F.Cu) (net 4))
 (segment (start 139.276 109.0373) (end 138.938 108.6993) (width 0.25) (layer F.Cu) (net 4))
 (segment (start 139.276 114.808) (end 139.7 114.808) (width 0.25) (layer F.Cu) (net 5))
 (segment (start 139.7 114.808) (end 140.97 113.538) (width 0.25) (layer F.Cu) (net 5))
 (segment (start 140.97 113.538) (end 140.97 108.6993) (width 0.25) (layer F.Cu) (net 5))
 (segment (start 130.81 98.298) (end 133.096 98.298) (width 0.25) (layer F.Cu) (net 6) (status 400000))
 (segment (start 135.89 99.822) (end 138.43 97.282) (width 0.25) (layer F.Cu) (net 6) (status 800000))
 (segment (start 134.62 99.822) (end 135.89 99.822) (width 0.25) (layer F.Cu) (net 6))
 (segment (start 133.096 98.298) (end 134.62 99.822) (width 0.25) (layer F.Cu) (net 6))
 (segment (start 133.942 114.996) (end 136.888 114.996) (width 0.25) (layer F.Cu) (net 7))
 (segment (start 136.888 114.996) (end 137.076 114.808) (width 0.25) (layer F.Cu) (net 7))
 (segment (start 137.076 114.808) (end 137.076 112.522) (width 0.25) (layer F.Cu) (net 7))
 (segment (start 131.826 117.264) (end 131.826 115.08) (width 0.25) (layer F.Cu) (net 8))
 (segment (start 131.826 115.08) (end 131.742 114.996) (width 0.25) (layer F.Cu) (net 8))
 (segment (start 129.3876 115.062) (end 131.676 115.062) (width 0.25) (layer F.Cu) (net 8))
 (segment (start 131.676 115.062) (end 131.742 114.996) (width 0.25) (layer F.Cu) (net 8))
 (segment (start 129.54 117.264) (end 129.54 117.094) (width 0.25) (layer F.Cu) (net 9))
 (segment (start 129.54 117.094) (end 128.6764 116.2304) (width 0.25) (layer F.Cu) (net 9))
 (segment (start 128.6764 116.2304) (end 128.6764 115.062) (width 0.25) (layer F.Cu) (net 9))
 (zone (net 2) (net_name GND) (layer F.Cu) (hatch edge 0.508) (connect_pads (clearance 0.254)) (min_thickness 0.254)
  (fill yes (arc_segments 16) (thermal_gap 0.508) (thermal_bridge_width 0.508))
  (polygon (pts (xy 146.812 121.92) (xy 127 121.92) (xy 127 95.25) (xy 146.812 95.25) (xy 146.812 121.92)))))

